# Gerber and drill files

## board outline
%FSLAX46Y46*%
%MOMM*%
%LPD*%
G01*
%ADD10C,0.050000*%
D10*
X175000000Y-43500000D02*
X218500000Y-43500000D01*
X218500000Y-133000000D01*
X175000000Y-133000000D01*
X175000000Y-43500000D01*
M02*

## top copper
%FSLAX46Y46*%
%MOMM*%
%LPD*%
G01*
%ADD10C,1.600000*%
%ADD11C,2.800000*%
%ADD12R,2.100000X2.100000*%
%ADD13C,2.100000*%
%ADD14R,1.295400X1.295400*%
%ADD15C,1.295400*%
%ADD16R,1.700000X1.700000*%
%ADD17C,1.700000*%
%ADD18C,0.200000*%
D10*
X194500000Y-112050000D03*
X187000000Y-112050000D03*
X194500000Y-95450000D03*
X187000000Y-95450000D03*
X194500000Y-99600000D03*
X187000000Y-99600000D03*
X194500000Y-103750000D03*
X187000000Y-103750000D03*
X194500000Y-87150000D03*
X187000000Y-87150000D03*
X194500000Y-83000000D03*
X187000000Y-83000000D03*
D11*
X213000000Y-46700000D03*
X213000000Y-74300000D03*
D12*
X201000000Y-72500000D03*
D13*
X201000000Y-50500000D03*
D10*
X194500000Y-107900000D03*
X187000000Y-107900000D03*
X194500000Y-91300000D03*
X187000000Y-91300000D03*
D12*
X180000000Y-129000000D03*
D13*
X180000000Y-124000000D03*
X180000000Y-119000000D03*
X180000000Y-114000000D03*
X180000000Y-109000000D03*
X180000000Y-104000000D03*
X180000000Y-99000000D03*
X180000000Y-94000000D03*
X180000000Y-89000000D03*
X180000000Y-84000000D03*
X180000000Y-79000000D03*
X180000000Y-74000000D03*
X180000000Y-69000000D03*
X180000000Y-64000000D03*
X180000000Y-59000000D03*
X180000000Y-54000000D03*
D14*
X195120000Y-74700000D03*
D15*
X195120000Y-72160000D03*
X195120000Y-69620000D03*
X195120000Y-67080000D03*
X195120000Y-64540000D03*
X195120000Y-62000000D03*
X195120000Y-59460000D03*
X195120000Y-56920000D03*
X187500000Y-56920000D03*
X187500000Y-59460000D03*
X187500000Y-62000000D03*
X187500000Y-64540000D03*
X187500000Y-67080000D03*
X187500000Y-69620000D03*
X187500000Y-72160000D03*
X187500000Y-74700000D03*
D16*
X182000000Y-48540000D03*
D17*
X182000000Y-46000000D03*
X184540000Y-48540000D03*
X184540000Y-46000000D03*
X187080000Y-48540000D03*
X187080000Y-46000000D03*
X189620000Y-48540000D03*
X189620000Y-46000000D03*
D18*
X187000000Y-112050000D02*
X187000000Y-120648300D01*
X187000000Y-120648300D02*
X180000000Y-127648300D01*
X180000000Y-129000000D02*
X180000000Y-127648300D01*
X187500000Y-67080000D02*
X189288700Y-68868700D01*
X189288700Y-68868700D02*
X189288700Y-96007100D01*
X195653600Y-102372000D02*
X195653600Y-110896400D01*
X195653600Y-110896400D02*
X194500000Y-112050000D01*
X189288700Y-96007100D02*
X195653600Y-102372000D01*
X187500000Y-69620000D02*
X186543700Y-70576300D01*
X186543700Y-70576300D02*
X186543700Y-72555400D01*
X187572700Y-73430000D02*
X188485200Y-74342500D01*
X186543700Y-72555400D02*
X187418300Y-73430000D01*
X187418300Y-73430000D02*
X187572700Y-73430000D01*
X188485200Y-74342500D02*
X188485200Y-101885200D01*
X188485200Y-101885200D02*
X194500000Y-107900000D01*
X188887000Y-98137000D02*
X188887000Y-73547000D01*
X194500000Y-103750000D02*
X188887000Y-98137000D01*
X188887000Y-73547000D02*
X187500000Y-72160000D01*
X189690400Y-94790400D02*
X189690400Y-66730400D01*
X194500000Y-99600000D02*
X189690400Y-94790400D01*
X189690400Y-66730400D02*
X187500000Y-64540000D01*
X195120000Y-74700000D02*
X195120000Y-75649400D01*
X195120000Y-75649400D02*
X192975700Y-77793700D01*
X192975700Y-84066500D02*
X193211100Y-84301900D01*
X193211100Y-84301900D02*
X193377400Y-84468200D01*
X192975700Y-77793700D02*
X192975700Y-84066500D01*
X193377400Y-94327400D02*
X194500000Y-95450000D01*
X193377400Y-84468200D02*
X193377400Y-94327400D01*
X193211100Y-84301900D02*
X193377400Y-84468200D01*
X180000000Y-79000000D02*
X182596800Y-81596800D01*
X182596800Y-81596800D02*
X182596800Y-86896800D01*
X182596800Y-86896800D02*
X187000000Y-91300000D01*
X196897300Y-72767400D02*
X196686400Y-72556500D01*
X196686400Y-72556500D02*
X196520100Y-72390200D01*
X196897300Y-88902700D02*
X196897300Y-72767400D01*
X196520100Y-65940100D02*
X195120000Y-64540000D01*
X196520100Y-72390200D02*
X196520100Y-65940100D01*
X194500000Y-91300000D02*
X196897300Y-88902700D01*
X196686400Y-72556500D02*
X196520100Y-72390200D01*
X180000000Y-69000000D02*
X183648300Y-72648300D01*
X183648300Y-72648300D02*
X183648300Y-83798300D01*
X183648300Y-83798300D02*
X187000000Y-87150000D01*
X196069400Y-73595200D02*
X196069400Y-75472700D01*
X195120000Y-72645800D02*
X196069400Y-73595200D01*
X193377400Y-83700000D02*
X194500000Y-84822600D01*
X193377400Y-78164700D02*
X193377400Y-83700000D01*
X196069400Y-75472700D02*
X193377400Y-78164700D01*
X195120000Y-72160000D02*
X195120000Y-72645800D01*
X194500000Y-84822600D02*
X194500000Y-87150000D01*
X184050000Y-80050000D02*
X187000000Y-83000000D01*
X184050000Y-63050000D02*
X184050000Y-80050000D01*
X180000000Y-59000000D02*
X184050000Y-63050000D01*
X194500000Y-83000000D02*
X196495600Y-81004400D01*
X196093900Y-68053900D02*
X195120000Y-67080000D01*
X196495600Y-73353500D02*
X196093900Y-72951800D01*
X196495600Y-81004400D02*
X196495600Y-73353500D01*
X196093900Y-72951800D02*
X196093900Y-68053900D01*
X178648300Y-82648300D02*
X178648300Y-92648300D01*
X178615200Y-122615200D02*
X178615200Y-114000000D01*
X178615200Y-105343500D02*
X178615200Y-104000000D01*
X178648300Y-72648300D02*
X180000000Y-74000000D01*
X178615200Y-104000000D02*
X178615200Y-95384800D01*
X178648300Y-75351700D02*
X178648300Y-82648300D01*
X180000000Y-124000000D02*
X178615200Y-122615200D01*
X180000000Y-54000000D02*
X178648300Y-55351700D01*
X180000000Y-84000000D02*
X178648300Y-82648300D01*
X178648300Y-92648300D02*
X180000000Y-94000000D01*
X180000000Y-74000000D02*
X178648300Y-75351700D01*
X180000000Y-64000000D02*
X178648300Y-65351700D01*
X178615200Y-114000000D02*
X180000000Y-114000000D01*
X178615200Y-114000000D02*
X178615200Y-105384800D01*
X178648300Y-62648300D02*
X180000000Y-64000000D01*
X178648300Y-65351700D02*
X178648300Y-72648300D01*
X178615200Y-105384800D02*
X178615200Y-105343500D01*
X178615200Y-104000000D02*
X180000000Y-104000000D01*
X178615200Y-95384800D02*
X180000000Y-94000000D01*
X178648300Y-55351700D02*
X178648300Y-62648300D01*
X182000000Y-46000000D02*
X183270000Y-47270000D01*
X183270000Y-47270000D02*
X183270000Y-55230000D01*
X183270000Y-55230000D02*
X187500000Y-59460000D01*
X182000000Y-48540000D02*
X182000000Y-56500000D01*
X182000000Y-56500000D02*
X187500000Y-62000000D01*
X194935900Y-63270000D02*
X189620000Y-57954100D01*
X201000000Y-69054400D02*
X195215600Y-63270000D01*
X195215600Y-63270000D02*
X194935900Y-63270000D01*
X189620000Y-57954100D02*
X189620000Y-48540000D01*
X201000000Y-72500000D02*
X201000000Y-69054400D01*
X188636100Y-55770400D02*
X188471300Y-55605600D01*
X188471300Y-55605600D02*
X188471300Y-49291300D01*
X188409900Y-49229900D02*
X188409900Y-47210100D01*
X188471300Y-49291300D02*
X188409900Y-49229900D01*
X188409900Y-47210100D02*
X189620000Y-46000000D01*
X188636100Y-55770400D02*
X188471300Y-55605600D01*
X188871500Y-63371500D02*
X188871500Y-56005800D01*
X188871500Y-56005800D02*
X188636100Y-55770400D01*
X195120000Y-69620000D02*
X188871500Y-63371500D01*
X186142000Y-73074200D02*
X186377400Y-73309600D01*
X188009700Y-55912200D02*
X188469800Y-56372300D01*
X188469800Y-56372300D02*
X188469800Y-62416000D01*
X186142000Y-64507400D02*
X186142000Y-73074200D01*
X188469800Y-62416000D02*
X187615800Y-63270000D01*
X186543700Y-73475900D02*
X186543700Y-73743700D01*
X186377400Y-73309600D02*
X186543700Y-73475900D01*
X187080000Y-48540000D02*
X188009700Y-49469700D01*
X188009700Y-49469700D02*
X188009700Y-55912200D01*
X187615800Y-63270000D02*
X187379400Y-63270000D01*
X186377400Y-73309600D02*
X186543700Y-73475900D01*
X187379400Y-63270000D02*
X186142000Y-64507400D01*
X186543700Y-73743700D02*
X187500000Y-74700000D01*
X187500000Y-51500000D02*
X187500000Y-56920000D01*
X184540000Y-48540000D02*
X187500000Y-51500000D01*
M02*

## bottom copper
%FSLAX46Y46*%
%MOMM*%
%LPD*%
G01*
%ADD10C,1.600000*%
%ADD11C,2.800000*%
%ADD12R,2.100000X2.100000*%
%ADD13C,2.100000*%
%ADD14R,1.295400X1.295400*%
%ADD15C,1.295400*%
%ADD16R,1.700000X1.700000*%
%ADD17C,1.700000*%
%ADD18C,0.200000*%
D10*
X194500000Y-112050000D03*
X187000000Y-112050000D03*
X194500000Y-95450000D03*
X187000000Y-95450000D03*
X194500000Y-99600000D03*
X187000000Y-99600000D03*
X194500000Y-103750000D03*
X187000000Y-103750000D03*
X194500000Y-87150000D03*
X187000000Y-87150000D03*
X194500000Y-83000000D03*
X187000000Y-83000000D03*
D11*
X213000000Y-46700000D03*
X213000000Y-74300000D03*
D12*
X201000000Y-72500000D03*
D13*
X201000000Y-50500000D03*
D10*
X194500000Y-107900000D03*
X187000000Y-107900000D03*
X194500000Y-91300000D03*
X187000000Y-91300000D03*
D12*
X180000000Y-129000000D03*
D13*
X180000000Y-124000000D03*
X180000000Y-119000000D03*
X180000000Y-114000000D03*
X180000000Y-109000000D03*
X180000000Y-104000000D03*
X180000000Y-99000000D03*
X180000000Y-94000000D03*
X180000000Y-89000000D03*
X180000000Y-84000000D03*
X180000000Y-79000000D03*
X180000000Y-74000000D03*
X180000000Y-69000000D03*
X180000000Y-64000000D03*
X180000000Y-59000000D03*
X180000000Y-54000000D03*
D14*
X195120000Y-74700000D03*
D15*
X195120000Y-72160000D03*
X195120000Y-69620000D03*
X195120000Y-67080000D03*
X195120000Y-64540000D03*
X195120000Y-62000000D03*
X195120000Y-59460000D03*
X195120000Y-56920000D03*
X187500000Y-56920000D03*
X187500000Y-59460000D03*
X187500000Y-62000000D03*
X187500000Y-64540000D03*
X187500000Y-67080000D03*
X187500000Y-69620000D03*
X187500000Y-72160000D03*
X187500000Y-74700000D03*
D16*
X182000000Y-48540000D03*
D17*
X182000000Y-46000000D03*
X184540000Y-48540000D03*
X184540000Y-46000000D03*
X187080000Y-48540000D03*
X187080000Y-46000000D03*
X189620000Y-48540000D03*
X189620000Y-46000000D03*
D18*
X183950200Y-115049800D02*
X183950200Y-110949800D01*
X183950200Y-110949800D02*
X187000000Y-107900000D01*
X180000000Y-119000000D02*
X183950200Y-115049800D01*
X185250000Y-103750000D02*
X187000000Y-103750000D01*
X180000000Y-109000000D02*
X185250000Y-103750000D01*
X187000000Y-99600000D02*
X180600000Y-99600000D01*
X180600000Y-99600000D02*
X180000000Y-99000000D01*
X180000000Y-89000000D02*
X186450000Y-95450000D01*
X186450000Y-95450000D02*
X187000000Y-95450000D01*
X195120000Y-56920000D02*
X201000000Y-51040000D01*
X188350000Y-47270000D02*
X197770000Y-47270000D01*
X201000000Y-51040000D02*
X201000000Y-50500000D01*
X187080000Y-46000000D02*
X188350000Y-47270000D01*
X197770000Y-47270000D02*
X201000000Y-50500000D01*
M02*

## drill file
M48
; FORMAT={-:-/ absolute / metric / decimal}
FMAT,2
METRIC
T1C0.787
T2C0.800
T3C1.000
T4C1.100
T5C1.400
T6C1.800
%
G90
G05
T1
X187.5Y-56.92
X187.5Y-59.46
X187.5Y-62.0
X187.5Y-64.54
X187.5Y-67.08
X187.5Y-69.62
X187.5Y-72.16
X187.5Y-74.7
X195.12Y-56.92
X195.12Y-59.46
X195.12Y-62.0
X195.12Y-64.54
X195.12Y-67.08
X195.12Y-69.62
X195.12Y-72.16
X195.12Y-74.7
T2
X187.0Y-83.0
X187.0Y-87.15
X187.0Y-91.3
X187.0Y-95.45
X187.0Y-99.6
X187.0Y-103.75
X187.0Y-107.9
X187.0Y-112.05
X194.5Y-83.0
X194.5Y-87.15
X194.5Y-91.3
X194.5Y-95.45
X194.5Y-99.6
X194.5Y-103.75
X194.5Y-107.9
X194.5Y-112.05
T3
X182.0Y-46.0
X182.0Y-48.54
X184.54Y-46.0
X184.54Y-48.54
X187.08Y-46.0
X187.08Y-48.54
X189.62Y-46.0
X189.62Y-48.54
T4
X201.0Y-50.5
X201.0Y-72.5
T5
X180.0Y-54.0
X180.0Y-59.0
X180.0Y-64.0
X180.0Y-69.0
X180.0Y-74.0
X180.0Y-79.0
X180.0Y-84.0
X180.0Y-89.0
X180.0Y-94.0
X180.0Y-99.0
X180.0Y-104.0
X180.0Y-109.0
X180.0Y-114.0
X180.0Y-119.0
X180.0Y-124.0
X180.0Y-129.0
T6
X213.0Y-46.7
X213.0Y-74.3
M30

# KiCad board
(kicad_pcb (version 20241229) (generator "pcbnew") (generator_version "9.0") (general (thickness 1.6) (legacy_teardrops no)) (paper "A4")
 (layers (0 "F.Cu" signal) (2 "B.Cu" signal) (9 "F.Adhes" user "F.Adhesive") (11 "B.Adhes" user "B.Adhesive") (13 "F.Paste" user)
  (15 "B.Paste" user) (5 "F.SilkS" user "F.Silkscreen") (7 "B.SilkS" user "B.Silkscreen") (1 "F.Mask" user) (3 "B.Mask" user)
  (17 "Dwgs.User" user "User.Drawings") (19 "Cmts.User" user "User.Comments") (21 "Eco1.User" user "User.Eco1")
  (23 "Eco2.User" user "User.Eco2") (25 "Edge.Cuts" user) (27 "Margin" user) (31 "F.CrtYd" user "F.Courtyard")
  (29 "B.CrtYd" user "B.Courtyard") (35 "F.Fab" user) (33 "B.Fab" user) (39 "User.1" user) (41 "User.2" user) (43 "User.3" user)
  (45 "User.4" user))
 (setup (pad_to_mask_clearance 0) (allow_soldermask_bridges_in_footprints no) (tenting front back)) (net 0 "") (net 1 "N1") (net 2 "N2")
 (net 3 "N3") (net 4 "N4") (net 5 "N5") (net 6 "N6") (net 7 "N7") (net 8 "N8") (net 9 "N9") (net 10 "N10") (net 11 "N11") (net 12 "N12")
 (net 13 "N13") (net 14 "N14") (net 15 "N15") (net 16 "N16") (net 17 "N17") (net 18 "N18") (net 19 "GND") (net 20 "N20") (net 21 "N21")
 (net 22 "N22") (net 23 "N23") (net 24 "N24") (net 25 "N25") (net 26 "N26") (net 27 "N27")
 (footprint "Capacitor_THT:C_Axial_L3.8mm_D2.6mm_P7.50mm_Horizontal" (layer "F.Cu") (at 194.5 112.05 180)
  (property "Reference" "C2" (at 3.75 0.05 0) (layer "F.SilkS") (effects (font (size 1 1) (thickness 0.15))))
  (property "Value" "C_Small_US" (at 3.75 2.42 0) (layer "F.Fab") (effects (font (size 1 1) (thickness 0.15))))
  (pad "1" thru_hole circle (at 0 0 180) (size 1.6 1.6) (drill 0.8) (layers "*.Cu" "*.Mask") (remove_unused_layers no) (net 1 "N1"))
  (pad "2" thru_hole circle (at 7.5 0 180) (size 1.6 1.6) (drill 0.8) (layers "*.Cu" "*.Mask") (remove_unused_layers no) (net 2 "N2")))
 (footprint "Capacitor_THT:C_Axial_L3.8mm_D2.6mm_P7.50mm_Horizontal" (layer "F.Cu") (at 194.5 95.45 180)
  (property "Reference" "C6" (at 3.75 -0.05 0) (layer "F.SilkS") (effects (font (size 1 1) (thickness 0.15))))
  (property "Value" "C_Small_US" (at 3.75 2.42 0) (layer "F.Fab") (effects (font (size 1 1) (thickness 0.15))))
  (pad "1" thru_hole circle (at 0 0 180) (size 1.6 1.6) (drill 0.8) (layers "*.Cu" "*.Mask") (remove_unused_layers no) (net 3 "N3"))
  (pad "2" thru_hole circle (at 7.5 0 180) (size 1.6 1.6) (drill 0.8) (layers "*.Cu" "*.Mask") (remove_unused_layers no) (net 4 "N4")))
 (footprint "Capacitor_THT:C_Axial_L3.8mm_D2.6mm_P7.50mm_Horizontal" (layer "F.Cu") (at 194.5 99.6 180)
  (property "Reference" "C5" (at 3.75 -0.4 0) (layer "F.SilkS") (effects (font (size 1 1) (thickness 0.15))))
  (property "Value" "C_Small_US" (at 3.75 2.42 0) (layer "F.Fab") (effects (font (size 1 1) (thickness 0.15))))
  (pad "1" thru_hole circle (at 0 0 180) (size 1.6 1.6) (drill 0.8) (layers "*.Cu" "*.Mask") (remove_unused_layers no) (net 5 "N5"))
  (pad "2" thru_hole circle (at 7.5 0 180) (size 1.6 1.6) (drill 0.8) (layers "*.Cu" "*.Mask") (remove_unused_layers no) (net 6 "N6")))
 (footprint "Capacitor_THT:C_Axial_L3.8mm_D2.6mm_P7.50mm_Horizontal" (layer "F.Cu") (at 194.5 103.75 180)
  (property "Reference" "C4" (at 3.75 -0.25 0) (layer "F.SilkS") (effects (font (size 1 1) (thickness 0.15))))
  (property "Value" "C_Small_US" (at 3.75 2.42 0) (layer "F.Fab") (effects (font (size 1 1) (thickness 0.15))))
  (pad "1" thru_hole circle (at 0 0 180) (size 1.6 1.6) (drill 0.8) (layers "*.Cu" "*.Mask") (remove_unused_layers no) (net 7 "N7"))
  (pad "2" thru_hole circle (at 7.5 0 180) (size 1.6 1.6) (drill 0.8) (layers "*.Cu" "*.Mask") (remove_unused_layers no) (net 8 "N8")))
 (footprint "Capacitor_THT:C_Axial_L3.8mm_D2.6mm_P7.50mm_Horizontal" (layer "F.Cu") (at 194.5 87.15 180)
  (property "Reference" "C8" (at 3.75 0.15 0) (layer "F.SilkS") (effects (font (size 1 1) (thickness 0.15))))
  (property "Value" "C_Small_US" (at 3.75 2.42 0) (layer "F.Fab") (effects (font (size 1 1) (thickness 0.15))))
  (pad "1" thru_hole circle (at 0 0 180) (size 1.6 1.6) (drill 0.8) (layers "*.Cu" "*.Mask") (remove_unused_layers no) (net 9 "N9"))
  (pad "2" thru_hole circle (at 7.5 0 180) (size 1.6 1.6) (drill 0.8) (layers "*.Cu" "*.Mask") (remove_unused_layers no) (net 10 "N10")))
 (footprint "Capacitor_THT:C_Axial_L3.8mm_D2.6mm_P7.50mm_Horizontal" (layer "F.Cu") (at 194.5 83 180)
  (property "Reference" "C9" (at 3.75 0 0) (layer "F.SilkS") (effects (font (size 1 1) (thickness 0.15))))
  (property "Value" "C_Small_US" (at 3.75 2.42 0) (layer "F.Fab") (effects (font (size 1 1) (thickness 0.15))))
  (pad "1" thru_hole circle (at 0 0 180) (size 1.6 1.6) (drill 0.8) (layers "*.Cu" "*.Mask") (remove_unused_layers no) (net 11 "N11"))
  (pad "2" thru_hole circle (at 7.5 0 180) (size 1.6 1.6) (drill 0.8) (layers "*.Cu" "*.Mask") (remove_unused_layers no) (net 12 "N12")))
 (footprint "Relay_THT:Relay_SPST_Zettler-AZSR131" (layer "F.Cu") (at 201 72.5 90)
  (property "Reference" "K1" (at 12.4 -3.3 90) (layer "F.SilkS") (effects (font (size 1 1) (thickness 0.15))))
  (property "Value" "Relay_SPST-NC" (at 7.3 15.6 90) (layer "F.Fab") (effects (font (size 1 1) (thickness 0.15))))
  (pad "13" thru_hole circle (at 25.8 12 270) (size 2.8 2.8) (drill 1.8) (layers "*.Cu" "*.Mask") (remove_unused_layers no))
  (pad "14" thru_hole circle (at -1.8 12 270) (size 2.8 2.8) (drill 1.8) (layers "*.Cu" "*.Mask") (remove_unused_layers no))
  (pad "A1" thru_hole rect (at 0 0 270) (size 2.1 2.1) (drill 1.1) (layers "*.Cu" "*.Mask") (remove_unused_layers no) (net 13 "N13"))
  (pad "A2" thru_hole circle (at 22 0 270) (size 2.1 2.1) (drill 1.1) (layers "*.Cu" "*.Mask") (remove_unused_layers no) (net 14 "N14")))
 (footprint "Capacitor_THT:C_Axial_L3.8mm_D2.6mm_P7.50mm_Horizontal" (layer "F.Cu") (at 194.5 107.9 180)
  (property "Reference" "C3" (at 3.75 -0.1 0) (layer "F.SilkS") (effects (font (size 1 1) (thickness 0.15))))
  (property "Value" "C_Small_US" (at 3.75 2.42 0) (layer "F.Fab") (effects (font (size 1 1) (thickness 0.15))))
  (pad "1" thru_hole circle (at 0 0 180) (size 1.6 1.6) (drill 0.8) (layers "*.Cu" "*.Mask") (remove_unused_layers no) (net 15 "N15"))
  (pad "2" thru_hole circle (at 7.5 0 180) (size 1.6 1.6) (drill 0.8) (layers "*.Cu" "*.Mask") (remove_unused_layers no) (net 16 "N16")))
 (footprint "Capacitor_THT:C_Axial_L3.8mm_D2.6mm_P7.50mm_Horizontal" (layer "F.Cu") (at 194.5 91.3 180)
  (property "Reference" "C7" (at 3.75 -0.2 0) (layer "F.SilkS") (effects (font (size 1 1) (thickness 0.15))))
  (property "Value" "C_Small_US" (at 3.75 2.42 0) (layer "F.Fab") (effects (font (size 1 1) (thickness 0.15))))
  (pad "1" thru_hole circle (at 0 0 180) (size 1.6 1.6) (drill 0.8) (layers "*.Cu" "*.Mask") (remove_unused_layers no) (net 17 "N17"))
  (pad "2" thru_hole circle (at 7.5 0 180) (size 1.6 1.6) (drill 0.8) (layers "*.Cu" "*.Mask") (remove_unused_layers no) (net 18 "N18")))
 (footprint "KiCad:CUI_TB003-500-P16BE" (layer "F.Cu") (at 180 129 90)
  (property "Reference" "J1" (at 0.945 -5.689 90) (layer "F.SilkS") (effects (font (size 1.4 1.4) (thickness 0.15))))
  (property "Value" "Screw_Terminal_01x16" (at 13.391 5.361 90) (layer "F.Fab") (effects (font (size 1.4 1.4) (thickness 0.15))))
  (pad "1" thru_hole rect (at 0 0 90) (size 2.1 2.1) (drill 1.4) (layers "*.Cu" "*.Mask") (remove_unused_layers no) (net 2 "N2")
   (solder_mask_margin 0.102))
  (pad "2" thru_hole circle (at 5 0 90) (size 2.1 2.1) (drill 1.4) (layers "*.Cu" "*.Mask") (remove_unused_layers no) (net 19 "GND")
   (solder_mask_margin 0.102))
  (pad "3" thru_hole circle (at 10 0 90) (size 2.1 2.1) (drill 1.4) (layers "*.Cu" "*.Mask") (remove_unused_layers no) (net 16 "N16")
   (solder_mask_margin 0.102))
  (pad "4" thru_hole circle (at 15 0 90) (size 2.1 2.1) (drill 1.4) (layers "*.Cu" "*.Mask") (remove_unused_layers no) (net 19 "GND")
   (solder_mask_margin 0.102))
  (pad "5" thru_hole circle (at 20 0 90) (size 2.1 2.1) (drill 1.4) (layers "*.Cu" "*.Mask") (remove_unused_layers no) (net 8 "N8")
   (solder_mask_margin 0.102))
  (pad "6" thru_hole circle (at 25 0 90) (size 2.1 2.1) (drill 1.4) (layers "*.Cu" "*.Mask") (remove_unused_layers no) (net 19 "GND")
   (solder_mask_margin 0.102))
  (pad "7" thru_hole circle (at 30 0 90) (size 2.1 2.1) (drill 1.4) (layers "*.Cu" "*.Mask") (remove_unused_layers no) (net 6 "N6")
   (solder_mask_margin 0.102))
  (pad "8" thru_hole circle (at 35 0 90) (size 2.1 2.1) (drill 1.4) (layers "*.Cu" "*.Mask") (remove_unused_layers no) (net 19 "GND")
   (solder_mask_margin 0.102))
  (pad "9" thru_hole circle (at 40 0 90) (size 2.1 2.1) (drill 1.4) (layers "*.Cu" "*.Mask") (remove_unused_layers no) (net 4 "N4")
   (solder_mask_margin 0.102))
  (pad "10" thru_hole circle (at 45 0 90) (size 2.1 2.1) (drill 1.4) (layers "*.Cu" "*.Mask") (remove_unused_layers no) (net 19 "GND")
   (solder_mask_margin 0.102))
  (pad "11" thru_hole circle (at 50 0 90) (size 2.1 2.1) (drill 1.4) (layers "*.Cu" "*.Mask") (remove_unused_layers no) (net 18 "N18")
   (solder_mask_margin 0.102))
  (pad "12" thru_hole circle (at 55 0 90) (size 2.1 2.1) (drill 1.4) (layers "*.Cu" "*.Mask") (remove_unused_layers no) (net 19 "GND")
   (solder_mask_margin 0.102))
  (pad "13" thru_hole circle (at 60 0 90) (size 2.1 2.1) (drill 1.4) (layers "*.Cu" "*.Mask") (remove_unused_layers no) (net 10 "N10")
   (solder_mask_margin 0.102))
  (pad "14" thru_hole circle (at 65 0 90) (size 2.1 2.1) (drill 1.4) (layers "*.Cu" "*.Mask") (remove_unused_layers no) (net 19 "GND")
   (solder_mask_margin 0.102))
  (pad "15" thru_hole circle (at 70 0 90) (size 2.1 2.1) (drill 1.4) (layers "*.Cu" "*.Mask") (remove_unused_layers no) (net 12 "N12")
   (solder_mask_margin 0.102))
  (pad "16" thru_hole circle (at 75 0 90) (size 2.1 2.1) (drill 1.4) (layers "*.Cu" "*.Mask") (remove_unused_layers no) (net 19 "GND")
   (solder_mask_margin 0.102)))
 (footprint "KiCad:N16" (layer "F.Cu") (at 187.5 56.92 180)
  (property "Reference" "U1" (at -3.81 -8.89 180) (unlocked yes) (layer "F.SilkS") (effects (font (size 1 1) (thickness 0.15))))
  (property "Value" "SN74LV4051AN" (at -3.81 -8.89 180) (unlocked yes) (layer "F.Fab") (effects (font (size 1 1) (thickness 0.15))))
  (pad "1" thru_hole rect (at -7.62 -17.78 180) (size 1.2954 1.2954) (drill 0.7874) (layers "*.Cu" "*.Mask") (remove_unused_layers no)
   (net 3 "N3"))
  (pad "2" thru_hole circle (at -7.62 -15.24 180) (size 1.2954 1.2954) (drill 0.7874) (layers "*.Cu" "*.Mask") (remove_unused_layers no)
   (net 9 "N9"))
  (pad "3" thru_hole circle (at -7.62 -12.7 180) (size 1.2954 1.2954) (drill 0.7874) (layers "*.Cu" "*.Mask") (remove_unused_layers no)
   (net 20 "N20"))
  (pad "4" thru_hole circle (at -7.62 -10.16 180) (size 1.2954 1.2954) (drill 0.7874) (layers "*.Cu" "*.Mask") (remove_unused_layers no)
   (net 11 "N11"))
  (pad "5" thru_hole circle (at -7.62 -7.62 180) (size 1.2954 1.2954) (drill 0.7874) (layers "*.Cu" "*.Mask") (remove_unused_layers no)
   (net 17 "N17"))
  (pad "6" thru_hole circle (at -7.62 -5.08 180) (size 1.2954 1.2954) (drill 0.7874) (layers "*.Cu" "*.Mask") (remove_unused_layers no)
   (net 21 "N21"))
  (pad "7" thru_hole circle (at -7.62 -2.54 180) (size 1.2954 1.2954) (drill 0.7874) (layers "*.Cu" "*.Mask") (remove_unused_layers no)
   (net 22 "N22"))
  (pad "8" thru_hole circle (at -7.62 0 180) (size 1.2954 1.2954) (drill 0.7874) (layers "*.Cu" "*.Mask") (remove_unused_layers no)
   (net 14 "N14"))
  (pad "9" thru_hole circle (at 0 0 180) (size 1.2954 1.2954) (drill 0.7874) (layers "*.Cu" "*.Mask") (remove_unused_layers no)
   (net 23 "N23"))
  (pad "10" thru_hole circle (at 0 -2.54 180) (size 1.2954 1.2954) (drill 0.7874) (layers "*.Cu" "*.Mask") (remove_unused_layers no)
   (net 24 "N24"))
  (pad "11" thru_hole circle (at 0 -5.08 180) (size 1.2954 1.2954) (drill 0.7874) (layers "*.Cu" "*.Mask") (remove_unused_layers no)
   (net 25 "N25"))
  (pad "12" thru_hole circle (at 0 -7.62 180) (size 1.2954 1.2954) (drill 0.7874) (layers "*.Cu" "*.Mask") (remove_unused_layers no)
   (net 5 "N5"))
  (pad "13" thru_hole circle (at 0 -10.16 180) (size 1.2954 1.2954) (drill 0.7874) (layers "*.Cu" "*.Mask") (remove_unused_layers no)
   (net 1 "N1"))
  (pad "14" thru_hole circle (at 0 -12.7 180) (size 1.2954 1.2954) (drill 0.7874) (layers "*.Cu" "*.Mask") (remove_unused_layers no)
   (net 15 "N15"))
  (pad "15" thru_hole circle (at 0 -15.24 180) (size 1.2954 1.2954) (drill 0.7874) (layers "*.Cu" "*.Mask") (remove_unused_layers no)
   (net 7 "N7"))
  (pad "16" thru_hole circle (at 0 -17.78 180) (size 1.2954 1.2954) (drill 0.7874) (layers "*.Cu" "*.Mask") (remove_unused_layers no)
   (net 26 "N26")))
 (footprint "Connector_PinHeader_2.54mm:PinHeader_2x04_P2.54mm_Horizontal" (layer "F.Cu") (at 182 48.54 90)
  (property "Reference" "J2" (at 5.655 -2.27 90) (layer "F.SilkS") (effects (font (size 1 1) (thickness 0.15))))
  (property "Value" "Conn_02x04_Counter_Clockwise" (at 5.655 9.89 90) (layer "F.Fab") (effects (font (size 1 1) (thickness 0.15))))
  (pad "1" thru_hole rect (at 0 0 90) (size 1.7 1.7) (drill 1) (layers "*.Cu" "*.Mask") (remove_unused_layers no) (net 25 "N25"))
  (pad "2" thru_hole circle (at 2.54 0 90) (size 1.7 1.7) (drill 1) (layers "*.Cu" "*.Mask") (remove_unused_layers no) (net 24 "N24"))
  (pad "3" thru_hole circle (at 0 2.54 90) (size 1.7 1.7) (drill 1) (layers "*.Cu" "*.Mask") (remove_unused_layers no) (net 23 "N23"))
  (pad "4" thru_hole circle (at 2.54 2.54 90) (size 1.7 1.7) (drill 1) (layers "*.Cu" "*.Mask") (remove_unused_layers no) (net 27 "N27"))
  (pad "5" thru_hole circle (at 0 5.08 90) (size 1.7 1.7) (drill 1) (layers "*.Cu" "*.Mask") (remove_unused_layers no) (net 26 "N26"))
  (pad "6" thru_hole circle (at 2.54 5.08 90) (size 1.7 1.7) (drill 1) (layers "*.Cu" "*.Mask") (remove_unused_layers no) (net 14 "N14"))
  (pad "7" thru_hole circle (at 0 7.62 90) (size 1.7 1.7) (drill 1) (layers "*.Cu" "*.Mask") (remove_unused_layers no) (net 13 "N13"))
  (pad "8" thru_hole circle (at 2.54 7.62 90) (size 1.7 1.7) (drill 1) (layers "*.Cu" "*.Mask") (remove_unused_layers no) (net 20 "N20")))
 (gr_rect (start 175 43.5) (end 218.5 133) (stroke (width 0.05) (type default)) (fill no) (layer "Edge.Cuts"))
 (segment (start 187 112.05) (end 187 120.6483) (width 0.2) (layer "F.Cu") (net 2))
 (segment (start 187 120.6483) (end 180 127.6483) (width 0.2) (layer "F.Cu") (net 2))
 (segment (start 180 129) (end 180 127.6483) (width 0.2) (layer "F.Cu") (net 2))
 (segment (start 187.5 67.08) (end 189.2887 68.8687) (width 0.2) (layer "F.Cu") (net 1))
 (segment (start 189.2887 68.8687) (end 189.2887 96.0071) (width 0.2) (layer "F.Cu") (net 1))
 (segment (start 195.6536 102.372) (end 195.6536 110.8964) (width 0.2) (layer "F.Cu") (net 1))
 (segment (start 195.6536 110.8964) (end 194.5 112.05) (width 0.2) (layer "F.Cu") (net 1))
 (segment (start 189.2887 96.0071) (end 195.6536 102.372) (width 0.2) (layer "F.Cu") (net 1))
 (segment (start 187.5 69.62) (end 186.5437 70.5763) (width 0.2) (layer "F.Cu") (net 15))
 (segment (start 186.5437 70.5763) (end 186.5437 72.5554) (width 0.2) (layer "F.Cu") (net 15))
 (segment (start 187.5727 73.43) (end 188.4852 74.3425) (width 0.2) (layer "F.Cu") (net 15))
 (segment (start 186.5437 72.5554) (end 187.4183 73.43) (width 0.2) (layer "F.Cu") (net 15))
 (segment (start 187.4183 73.43) (end 187.5727 73.43) (width 0.2) (layer "F.Cu") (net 15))
 (segment (start 188.4852 74.3425) (end 188.4852 101.8852) (width 0.2) (layer "F.Cu") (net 15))
 (segment (start 188.4852 101.8852) (end 194.5 107.9) (width 0.2) (layer "F.Cu") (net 15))
 (segment (start 183.9502 115.0498) (end 183.9502 110.9498) (width 0.2) (layer "B.Cu") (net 16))
 (segment (start 183.9502 110.9498) (end 187 107.9) (width 0.2) (layer "B.Cu") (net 16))
 (segment (start 180 119) (end 183.9502 115.0498) (width 0.2) (layer "B.Cu") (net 16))
 (segment (start 188.887 98.137) (end 188.887 73.547) (width 0.2) (layer "F.Cu") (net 7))
 (segment (start 194.5 103.75) (end 188.887 98.137) (width 0.2) (layer "F.Cu") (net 7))
 (segment (start 188.887 73.547) (end 187.5 72.16) (width 0.2) (layer "F.Cu") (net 7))
 (segment (start 185.25 103.75) (end 187 103.75) (width 0.2) (layer "B.Cu") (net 8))
 (segment (start 180 109) (end 185.25 103.75) (width 0.2) (layer "B.Cu") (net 8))
 (segment (start 189.6904 94.7904) (end 189.6904 66.7304) (width 0.2) (layer "F.Cu") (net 5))
 (segment (start 194.5 99.6) (end 189.6904 94.7904) (width 0.2) (layer "F.Cu") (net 5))
 (segment (start 189.6904 66.7304) (end 187.5 64.54) (width 0.2) (layer "F.Cu") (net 5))
 (segment (start 187 99.6) (end 180.6 99.6) (width 0.2) (layer "B.Cu") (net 6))
 (segment (start 180.6 99.6) (end 180 99) (width 0.2) (layer "B.Cu") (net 6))
 (segment (start 180 89) (end 186.45 95.45) (width 0.2) (layer "B.Cu") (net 4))
 (segment (start 186.45 95.45) (end 187 95.45) (width 0.2) (layer "B.Cu") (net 4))
 (segment (start 195.12 74.7) (end 195.12 75.6494) (width 0.2) (layer "F.Cu") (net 3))
 (segment (start 195.12 75.6494) (end 192.9757 77.7937) (width 0.2) (layer "F.Cu") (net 3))
 (segment (start 192.9757 84.0665) (end 193.2111 84.3019) (width 0.2) (layer "F.Cu") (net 3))
 (segment (start 193.2111 84.3019) (end 193.3774 84.4682) (width 0.2) (layer "F.Cu") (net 3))
 (segment (start 192.9757 77.7937) (end 192.9757 84.0665) (width 0.2) (layer "F.Cu") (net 3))
 (segment (start 193.3774 94.3274) (end 194.5 95.45) (width 0.2) (layer "F.Cu") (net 3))
 (segment (start 193.3774 84.4682) (end 193.3774 94.3274) (width 0.2) (layer "F.Cu") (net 3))
 (segment (start 193.2111 84.3019) (end 193.3774 84.4682) (width 0.2) (layer "F.Cu") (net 3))
 (segment (start 180 79) (end 182.5968 81.5968) (width 0.2) (layer "F.Cu") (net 18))
 (segment (start 182.5968 81.5968) (end 182.5968 86.8968) (width 0.2) (layer "F.Cu") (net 18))
 (segment (start 182.5968 86.8968) (end 187 91.3) (width 0.2) (layer "F.Cu") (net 18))
 (segment (start 196.8973 72.7674) (end 196.6864 72.5565) (width 0.2) (layer "F.Cu") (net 17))
 (segment (start 196.6864 72.5565) (end 196.5201 72.3902) (width 0.2) (layer "F.Cu") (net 17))
 (segment (start 196.8973 88.9027) (end 196.8973 72.7674) (width 0.2) (layer "F.Cu") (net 17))
 (segment (start 196.5201 65.9401) (end 195.12 64.54) (width 0.2) (layer "F.Cu") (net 17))
 (segment (start 196.5201 72.3902) (end 196.5201 65.9401) (width 0.2) (layer "F.Cu") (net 17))
 (segment (start 194.5 91.3) (end 196.8973 88.9027) (width 0.2) (layer "F.Cu") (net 17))
 (segment (start 196.6864 72.5565) (end 196.5201 72.3902) (width 0.2) (layer "F.Cu") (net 17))
 (segment (start 180 69) (end 183.6483 72.6483) (width 0.2) (layer "F.Cu") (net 10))
 (segment (start 183.6483 72.6483) (end 183.6483 83.7983) (width 0.2) (layer "F.Cu") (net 10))
 (segment (start 183.6483 83.7983) (end 187 87.15) (width 0.2) (layer "F.Cu") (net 10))
 (segment (start 196.0694 73.5952) (end 196.0694 75.4727) (width 0.2) (layer "F.Cu") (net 9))
 (segment (start 195.12 72.6458) (end 196.0694 73.5952) (width 0.2) (layer "F.Cu") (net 9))
 (segment (start 193.3774 83.7) (end 194.5 84.8226) (width 0.2) (layer "F.Cu") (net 9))
 (segment (start 193.3774 78.1647) (end 193.3774 83.7) (width 0.2) (layer "F.Cu") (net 9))
 (segment (start 196.0694 75.4727) (end 193.3774 78.1647) (width 0.2) (layer "F.Cu") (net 9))
 (segment (start 195.12 72.16) (end 195.12 72.6458) (width 0.2) (layer "F.Cu") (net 9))
 (segment (start 194.5 84.8226) (end 194.5 87.15) (width 0.2) (layer "F.Cu") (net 9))
 (segment (start 184.05 80.05) (end 187 83) (width 0.2) (layer "F.Cu") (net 12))
 (segment (start 184.05 63.05) (end 184.05 80.05) (width 0.2) (layer "F.Cu") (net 12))
 (segment (start 180 59) (end 184.05 63.05) (width 0.2) (layer "F.Cu") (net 12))
 (segment (start 194.5 83) (end 196.4956 81.0044) (width 0.2) (layer "F.Cu") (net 11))
 (segment (start 196.0939 68.0539) (end 195.12 67.08) (width 0.2) (layer "F.Cu") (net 11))
 (segment (start 196.4956 73.3535) (end 196.0939 72.9518) (width 0.2) (layer "F.Cu") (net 11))
 (segment (start 196.4956 81.0044) (end 196.4956 73.3535) (width 0.2) (layer "F.Cu") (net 11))
 (segment (start 196.0939 72.9518) (end 196.0939 68.0539) (width 0.2) (layer "F.Cu") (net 11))
 (segment (start 178.6483 82.6483) (end 178.6483 92.6483) (width 0.2) (layer "F.Cu") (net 19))
 (segment (start 178.6152 122.6152) (end 178.6152 114) (width 0.2) (layer "F.Cu") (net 19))
 (segment (start 178.6152 105.3435) (end 178.6152 104) (width 0.2) (layer "F.Cu") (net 19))
 (segment (start 178.6483 72.6483) (end 180 74) (width 0.2) (layer "F.Cu") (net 19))
 (segment (start 178.6152 104) (end 178.6152 95.3848) (width 0.2) (layer "F.Cu") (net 19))
 (segment (start 178.6483 75.3517) (end 178.6483 82.6483) (width 0.2) (layer "F.Cu") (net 19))
 (segment (start 180 124) (end 178.6152 122.6152) (width 0.2) (layer "F.Cu") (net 19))
 (segment (start 180 54) (end 178.6483 55.3517) (width 0.2) (layer "F.Cu") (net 19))
 (segment (start 180 84) (end 178.6483 82.6483) (width 0.2) (layer "F.Cu") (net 19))
 (segment (start 178.6483 92.6483) (end 180 94) (width 0.2) (layer "F.Cu") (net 19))
 (segment (start 180 74) (end 178.6483 75.3517) (width 0.2) (layer "F.Cu") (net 19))
 (segment (start 180 64) (end 178.6483 65.3517) (width 0.2) (layer "F.Cu") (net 19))
 (segment (start 178.6152 114) (end 180 114) (width 0.2) (layer "F.Cu") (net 19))
 (segment (start 178.6152 114) (end 178.6152 105.3848) (width 0.2) (layer "F.Cu") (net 19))
 (segment (start 178.6483 62.6483) (end 180 64) (width 0.2) (layer "F.Cu") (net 19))
 (segment (start 178.6483 65.3517) (end 178.6483 72.6483) (width 0.2) (layer "F.Cu") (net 19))
 (segment (start 178.6152 105.3848) (end 178.6152 105.3435) (width 0.2) (layer "F.Cu") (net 19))
 (segment (start 178.6152 104) (end 180 104) (width 0.2) (layer "F.Cu") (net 19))
 (segment (start 178.6152 95.3848) (end 180 94) (width 0.2) (layer "F.Cu") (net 19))
 (segment (start 178.6483 55.3517) (end 178.6483 62.6483) (width 0.2) (layer "F.Cu") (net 19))
 (segment (start 182 46) (end 183.27 47.27) (width 0.2) (layer "F.Cu") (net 24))
 (segment (start 183.27 47.27) (end 183.27 55.23) (width 0.2) (layer "F.Cu") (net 24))
 (segment (start 183.27 55.23) (end 187.5 59.46) (width 0.2) (layer "F.Cu") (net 24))
 (segment (start 182 48.54) (end 182 56.5) (width 0.2) (layer "F.Cu") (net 25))
 (segment (start 182 56.5) (end 187.5 62) (width 0.2) (layer "F.Cu") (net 25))
 (segment (start 194.9359 63.27) (end 189.62 57.9541) (width 0.2) (layer "F.Cu") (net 13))
 (segment (start 201 69.0544) (end 195.2156 63.27) (width 0.2) (layer "F.Cu") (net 13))
 (segment (start 195.2156 63.27) (end 194.9359 63.27) (width 0.2) (layer "F.Cu") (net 13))
 (segment (start 189.62 57.9541) (end 189.62 48.54) (width 0.2) (layer "F.Cu") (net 13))
 (segment (start 201 72.5) (end 201 69.0544) (width 0.2) (layer "F.Cu") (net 13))
 (segment (start 188.6361 55.7704) (end 188.4713 55.6056) (width 0.2) (layer "F.Cu") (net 20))
 (segment (start 188.4713 55.6056) (end 188.4713 49.2913) (width 0.2) (layer "F.Cu") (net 20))
 (segment (start 188.4099 49.2299) (end 188.4099 47.2101) (width 0.2) (layer "F.Cu") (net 20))
 (segment (start 188.4713 49.2913) (end 188.4099 49.2299) (width 0.2) (layer "F.Cu") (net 20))
 (segment (start 188.4099 47.2101) (end 189.62 46) (width 0.2) (layer "F.Cu") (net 20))
 (segment (start 188.6361 55.7704) (end 188.4713 55.6056) (width 0.2) (layer "F.Cu") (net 20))
 (segment (start 188.8715 63.3715) (end 188.8715 56.0058) (width 0.2) (layer "F.Cu") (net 20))
 (segment (start 188.8715 56.0058) (end 188.6361 55.7704) (width 0.2) (layer "F.Cu") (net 20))
 (segment (start 195.12 69.62) (end 188.8715 63.3715) (width 0.2) (layer "F.Cu") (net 20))
 (segment (start 186.142 73.0742) (end 186.3774 73.3096) (width 0.2) (layer "F.Cu") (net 26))
 (segment (start 188.0097 55.9122) (end 188.4698 56.3723) (width 0.2) (layer "F.Cu") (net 26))
 (segment (start 188.4698 56.3723) (end 188.4698 62.416) (width 0.2) (layer "F.Cu") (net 26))
 (segment (start 186.142 64.5074) (end 186.142 73.0742) (width 0.2) (layer "F.Cu") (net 26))
 (segment (start 188.4698 62.416) (end 187.6158 63.27) (width 0.2) (layer "F.Cu") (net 26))
 (segment (start 186.5437 73.4759) (end 186.5437 73.7437) (width 0.2) (layer "F.Cu") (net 26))
 (segment (start 186.3774 73.3096) (end 186.5437 73.4759) (width 0.2) (layer "F.Cu") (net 26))
 (segment (start 187.08 48.54) (end 188.0097 49.4697) (width 0.2) (layer "F.Cu") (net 26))
 (segment (start 188.0097 49.4697) (end 188.0097 55.9122) (width 0.2) (layer "F.Cu") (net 26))
 (segment (start 187.6158 63.27) (end 187.3794 63.27) (width 0.2) (layer "F.Cu") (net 26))
 (segment (start 186.3774 73.3096) (end 186.5437 73.4759) (width 0.2) (layer "F.Cu") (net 26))
 (segment (start 187.3794 63.27) (end 186.142 64.5074) (width 0.2) (layer "F.Cu") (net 26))
 (segment (start 186.5437 73.7437) (end 187.5 74.7) (width 0.2) (layer "F.Cu") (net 26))
 (segment (start 195.12 56.92) (end 201 51.04) (width 0.2) (layer "B.Cu") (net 14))
 (segment (start 188.35 47.27) (end 197.77 47.27) (width 0.2) (layer "B.Cu") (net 14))
 (segment (start 201 51.04) (end 201 50.5) (width 0.2) (layer "B.Cu") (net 14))
 (segment (start 187.08 46) (end 188.35 47.27) (width 0.2) (layer "B.Cu") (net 14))
 (segment (start 197.77 47.27) (end 201 50.5) (width 0.2) (layer "B.Cu") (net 14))
 (segment (start 187.5 51.5) (end 187.5 56.92) (width 0.2) (layer "F.Cu") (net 23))
 (segment (start 184.54 48.54) (end 187.5 51.5) (width 0.2) (layer "F.Cu") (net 23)))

